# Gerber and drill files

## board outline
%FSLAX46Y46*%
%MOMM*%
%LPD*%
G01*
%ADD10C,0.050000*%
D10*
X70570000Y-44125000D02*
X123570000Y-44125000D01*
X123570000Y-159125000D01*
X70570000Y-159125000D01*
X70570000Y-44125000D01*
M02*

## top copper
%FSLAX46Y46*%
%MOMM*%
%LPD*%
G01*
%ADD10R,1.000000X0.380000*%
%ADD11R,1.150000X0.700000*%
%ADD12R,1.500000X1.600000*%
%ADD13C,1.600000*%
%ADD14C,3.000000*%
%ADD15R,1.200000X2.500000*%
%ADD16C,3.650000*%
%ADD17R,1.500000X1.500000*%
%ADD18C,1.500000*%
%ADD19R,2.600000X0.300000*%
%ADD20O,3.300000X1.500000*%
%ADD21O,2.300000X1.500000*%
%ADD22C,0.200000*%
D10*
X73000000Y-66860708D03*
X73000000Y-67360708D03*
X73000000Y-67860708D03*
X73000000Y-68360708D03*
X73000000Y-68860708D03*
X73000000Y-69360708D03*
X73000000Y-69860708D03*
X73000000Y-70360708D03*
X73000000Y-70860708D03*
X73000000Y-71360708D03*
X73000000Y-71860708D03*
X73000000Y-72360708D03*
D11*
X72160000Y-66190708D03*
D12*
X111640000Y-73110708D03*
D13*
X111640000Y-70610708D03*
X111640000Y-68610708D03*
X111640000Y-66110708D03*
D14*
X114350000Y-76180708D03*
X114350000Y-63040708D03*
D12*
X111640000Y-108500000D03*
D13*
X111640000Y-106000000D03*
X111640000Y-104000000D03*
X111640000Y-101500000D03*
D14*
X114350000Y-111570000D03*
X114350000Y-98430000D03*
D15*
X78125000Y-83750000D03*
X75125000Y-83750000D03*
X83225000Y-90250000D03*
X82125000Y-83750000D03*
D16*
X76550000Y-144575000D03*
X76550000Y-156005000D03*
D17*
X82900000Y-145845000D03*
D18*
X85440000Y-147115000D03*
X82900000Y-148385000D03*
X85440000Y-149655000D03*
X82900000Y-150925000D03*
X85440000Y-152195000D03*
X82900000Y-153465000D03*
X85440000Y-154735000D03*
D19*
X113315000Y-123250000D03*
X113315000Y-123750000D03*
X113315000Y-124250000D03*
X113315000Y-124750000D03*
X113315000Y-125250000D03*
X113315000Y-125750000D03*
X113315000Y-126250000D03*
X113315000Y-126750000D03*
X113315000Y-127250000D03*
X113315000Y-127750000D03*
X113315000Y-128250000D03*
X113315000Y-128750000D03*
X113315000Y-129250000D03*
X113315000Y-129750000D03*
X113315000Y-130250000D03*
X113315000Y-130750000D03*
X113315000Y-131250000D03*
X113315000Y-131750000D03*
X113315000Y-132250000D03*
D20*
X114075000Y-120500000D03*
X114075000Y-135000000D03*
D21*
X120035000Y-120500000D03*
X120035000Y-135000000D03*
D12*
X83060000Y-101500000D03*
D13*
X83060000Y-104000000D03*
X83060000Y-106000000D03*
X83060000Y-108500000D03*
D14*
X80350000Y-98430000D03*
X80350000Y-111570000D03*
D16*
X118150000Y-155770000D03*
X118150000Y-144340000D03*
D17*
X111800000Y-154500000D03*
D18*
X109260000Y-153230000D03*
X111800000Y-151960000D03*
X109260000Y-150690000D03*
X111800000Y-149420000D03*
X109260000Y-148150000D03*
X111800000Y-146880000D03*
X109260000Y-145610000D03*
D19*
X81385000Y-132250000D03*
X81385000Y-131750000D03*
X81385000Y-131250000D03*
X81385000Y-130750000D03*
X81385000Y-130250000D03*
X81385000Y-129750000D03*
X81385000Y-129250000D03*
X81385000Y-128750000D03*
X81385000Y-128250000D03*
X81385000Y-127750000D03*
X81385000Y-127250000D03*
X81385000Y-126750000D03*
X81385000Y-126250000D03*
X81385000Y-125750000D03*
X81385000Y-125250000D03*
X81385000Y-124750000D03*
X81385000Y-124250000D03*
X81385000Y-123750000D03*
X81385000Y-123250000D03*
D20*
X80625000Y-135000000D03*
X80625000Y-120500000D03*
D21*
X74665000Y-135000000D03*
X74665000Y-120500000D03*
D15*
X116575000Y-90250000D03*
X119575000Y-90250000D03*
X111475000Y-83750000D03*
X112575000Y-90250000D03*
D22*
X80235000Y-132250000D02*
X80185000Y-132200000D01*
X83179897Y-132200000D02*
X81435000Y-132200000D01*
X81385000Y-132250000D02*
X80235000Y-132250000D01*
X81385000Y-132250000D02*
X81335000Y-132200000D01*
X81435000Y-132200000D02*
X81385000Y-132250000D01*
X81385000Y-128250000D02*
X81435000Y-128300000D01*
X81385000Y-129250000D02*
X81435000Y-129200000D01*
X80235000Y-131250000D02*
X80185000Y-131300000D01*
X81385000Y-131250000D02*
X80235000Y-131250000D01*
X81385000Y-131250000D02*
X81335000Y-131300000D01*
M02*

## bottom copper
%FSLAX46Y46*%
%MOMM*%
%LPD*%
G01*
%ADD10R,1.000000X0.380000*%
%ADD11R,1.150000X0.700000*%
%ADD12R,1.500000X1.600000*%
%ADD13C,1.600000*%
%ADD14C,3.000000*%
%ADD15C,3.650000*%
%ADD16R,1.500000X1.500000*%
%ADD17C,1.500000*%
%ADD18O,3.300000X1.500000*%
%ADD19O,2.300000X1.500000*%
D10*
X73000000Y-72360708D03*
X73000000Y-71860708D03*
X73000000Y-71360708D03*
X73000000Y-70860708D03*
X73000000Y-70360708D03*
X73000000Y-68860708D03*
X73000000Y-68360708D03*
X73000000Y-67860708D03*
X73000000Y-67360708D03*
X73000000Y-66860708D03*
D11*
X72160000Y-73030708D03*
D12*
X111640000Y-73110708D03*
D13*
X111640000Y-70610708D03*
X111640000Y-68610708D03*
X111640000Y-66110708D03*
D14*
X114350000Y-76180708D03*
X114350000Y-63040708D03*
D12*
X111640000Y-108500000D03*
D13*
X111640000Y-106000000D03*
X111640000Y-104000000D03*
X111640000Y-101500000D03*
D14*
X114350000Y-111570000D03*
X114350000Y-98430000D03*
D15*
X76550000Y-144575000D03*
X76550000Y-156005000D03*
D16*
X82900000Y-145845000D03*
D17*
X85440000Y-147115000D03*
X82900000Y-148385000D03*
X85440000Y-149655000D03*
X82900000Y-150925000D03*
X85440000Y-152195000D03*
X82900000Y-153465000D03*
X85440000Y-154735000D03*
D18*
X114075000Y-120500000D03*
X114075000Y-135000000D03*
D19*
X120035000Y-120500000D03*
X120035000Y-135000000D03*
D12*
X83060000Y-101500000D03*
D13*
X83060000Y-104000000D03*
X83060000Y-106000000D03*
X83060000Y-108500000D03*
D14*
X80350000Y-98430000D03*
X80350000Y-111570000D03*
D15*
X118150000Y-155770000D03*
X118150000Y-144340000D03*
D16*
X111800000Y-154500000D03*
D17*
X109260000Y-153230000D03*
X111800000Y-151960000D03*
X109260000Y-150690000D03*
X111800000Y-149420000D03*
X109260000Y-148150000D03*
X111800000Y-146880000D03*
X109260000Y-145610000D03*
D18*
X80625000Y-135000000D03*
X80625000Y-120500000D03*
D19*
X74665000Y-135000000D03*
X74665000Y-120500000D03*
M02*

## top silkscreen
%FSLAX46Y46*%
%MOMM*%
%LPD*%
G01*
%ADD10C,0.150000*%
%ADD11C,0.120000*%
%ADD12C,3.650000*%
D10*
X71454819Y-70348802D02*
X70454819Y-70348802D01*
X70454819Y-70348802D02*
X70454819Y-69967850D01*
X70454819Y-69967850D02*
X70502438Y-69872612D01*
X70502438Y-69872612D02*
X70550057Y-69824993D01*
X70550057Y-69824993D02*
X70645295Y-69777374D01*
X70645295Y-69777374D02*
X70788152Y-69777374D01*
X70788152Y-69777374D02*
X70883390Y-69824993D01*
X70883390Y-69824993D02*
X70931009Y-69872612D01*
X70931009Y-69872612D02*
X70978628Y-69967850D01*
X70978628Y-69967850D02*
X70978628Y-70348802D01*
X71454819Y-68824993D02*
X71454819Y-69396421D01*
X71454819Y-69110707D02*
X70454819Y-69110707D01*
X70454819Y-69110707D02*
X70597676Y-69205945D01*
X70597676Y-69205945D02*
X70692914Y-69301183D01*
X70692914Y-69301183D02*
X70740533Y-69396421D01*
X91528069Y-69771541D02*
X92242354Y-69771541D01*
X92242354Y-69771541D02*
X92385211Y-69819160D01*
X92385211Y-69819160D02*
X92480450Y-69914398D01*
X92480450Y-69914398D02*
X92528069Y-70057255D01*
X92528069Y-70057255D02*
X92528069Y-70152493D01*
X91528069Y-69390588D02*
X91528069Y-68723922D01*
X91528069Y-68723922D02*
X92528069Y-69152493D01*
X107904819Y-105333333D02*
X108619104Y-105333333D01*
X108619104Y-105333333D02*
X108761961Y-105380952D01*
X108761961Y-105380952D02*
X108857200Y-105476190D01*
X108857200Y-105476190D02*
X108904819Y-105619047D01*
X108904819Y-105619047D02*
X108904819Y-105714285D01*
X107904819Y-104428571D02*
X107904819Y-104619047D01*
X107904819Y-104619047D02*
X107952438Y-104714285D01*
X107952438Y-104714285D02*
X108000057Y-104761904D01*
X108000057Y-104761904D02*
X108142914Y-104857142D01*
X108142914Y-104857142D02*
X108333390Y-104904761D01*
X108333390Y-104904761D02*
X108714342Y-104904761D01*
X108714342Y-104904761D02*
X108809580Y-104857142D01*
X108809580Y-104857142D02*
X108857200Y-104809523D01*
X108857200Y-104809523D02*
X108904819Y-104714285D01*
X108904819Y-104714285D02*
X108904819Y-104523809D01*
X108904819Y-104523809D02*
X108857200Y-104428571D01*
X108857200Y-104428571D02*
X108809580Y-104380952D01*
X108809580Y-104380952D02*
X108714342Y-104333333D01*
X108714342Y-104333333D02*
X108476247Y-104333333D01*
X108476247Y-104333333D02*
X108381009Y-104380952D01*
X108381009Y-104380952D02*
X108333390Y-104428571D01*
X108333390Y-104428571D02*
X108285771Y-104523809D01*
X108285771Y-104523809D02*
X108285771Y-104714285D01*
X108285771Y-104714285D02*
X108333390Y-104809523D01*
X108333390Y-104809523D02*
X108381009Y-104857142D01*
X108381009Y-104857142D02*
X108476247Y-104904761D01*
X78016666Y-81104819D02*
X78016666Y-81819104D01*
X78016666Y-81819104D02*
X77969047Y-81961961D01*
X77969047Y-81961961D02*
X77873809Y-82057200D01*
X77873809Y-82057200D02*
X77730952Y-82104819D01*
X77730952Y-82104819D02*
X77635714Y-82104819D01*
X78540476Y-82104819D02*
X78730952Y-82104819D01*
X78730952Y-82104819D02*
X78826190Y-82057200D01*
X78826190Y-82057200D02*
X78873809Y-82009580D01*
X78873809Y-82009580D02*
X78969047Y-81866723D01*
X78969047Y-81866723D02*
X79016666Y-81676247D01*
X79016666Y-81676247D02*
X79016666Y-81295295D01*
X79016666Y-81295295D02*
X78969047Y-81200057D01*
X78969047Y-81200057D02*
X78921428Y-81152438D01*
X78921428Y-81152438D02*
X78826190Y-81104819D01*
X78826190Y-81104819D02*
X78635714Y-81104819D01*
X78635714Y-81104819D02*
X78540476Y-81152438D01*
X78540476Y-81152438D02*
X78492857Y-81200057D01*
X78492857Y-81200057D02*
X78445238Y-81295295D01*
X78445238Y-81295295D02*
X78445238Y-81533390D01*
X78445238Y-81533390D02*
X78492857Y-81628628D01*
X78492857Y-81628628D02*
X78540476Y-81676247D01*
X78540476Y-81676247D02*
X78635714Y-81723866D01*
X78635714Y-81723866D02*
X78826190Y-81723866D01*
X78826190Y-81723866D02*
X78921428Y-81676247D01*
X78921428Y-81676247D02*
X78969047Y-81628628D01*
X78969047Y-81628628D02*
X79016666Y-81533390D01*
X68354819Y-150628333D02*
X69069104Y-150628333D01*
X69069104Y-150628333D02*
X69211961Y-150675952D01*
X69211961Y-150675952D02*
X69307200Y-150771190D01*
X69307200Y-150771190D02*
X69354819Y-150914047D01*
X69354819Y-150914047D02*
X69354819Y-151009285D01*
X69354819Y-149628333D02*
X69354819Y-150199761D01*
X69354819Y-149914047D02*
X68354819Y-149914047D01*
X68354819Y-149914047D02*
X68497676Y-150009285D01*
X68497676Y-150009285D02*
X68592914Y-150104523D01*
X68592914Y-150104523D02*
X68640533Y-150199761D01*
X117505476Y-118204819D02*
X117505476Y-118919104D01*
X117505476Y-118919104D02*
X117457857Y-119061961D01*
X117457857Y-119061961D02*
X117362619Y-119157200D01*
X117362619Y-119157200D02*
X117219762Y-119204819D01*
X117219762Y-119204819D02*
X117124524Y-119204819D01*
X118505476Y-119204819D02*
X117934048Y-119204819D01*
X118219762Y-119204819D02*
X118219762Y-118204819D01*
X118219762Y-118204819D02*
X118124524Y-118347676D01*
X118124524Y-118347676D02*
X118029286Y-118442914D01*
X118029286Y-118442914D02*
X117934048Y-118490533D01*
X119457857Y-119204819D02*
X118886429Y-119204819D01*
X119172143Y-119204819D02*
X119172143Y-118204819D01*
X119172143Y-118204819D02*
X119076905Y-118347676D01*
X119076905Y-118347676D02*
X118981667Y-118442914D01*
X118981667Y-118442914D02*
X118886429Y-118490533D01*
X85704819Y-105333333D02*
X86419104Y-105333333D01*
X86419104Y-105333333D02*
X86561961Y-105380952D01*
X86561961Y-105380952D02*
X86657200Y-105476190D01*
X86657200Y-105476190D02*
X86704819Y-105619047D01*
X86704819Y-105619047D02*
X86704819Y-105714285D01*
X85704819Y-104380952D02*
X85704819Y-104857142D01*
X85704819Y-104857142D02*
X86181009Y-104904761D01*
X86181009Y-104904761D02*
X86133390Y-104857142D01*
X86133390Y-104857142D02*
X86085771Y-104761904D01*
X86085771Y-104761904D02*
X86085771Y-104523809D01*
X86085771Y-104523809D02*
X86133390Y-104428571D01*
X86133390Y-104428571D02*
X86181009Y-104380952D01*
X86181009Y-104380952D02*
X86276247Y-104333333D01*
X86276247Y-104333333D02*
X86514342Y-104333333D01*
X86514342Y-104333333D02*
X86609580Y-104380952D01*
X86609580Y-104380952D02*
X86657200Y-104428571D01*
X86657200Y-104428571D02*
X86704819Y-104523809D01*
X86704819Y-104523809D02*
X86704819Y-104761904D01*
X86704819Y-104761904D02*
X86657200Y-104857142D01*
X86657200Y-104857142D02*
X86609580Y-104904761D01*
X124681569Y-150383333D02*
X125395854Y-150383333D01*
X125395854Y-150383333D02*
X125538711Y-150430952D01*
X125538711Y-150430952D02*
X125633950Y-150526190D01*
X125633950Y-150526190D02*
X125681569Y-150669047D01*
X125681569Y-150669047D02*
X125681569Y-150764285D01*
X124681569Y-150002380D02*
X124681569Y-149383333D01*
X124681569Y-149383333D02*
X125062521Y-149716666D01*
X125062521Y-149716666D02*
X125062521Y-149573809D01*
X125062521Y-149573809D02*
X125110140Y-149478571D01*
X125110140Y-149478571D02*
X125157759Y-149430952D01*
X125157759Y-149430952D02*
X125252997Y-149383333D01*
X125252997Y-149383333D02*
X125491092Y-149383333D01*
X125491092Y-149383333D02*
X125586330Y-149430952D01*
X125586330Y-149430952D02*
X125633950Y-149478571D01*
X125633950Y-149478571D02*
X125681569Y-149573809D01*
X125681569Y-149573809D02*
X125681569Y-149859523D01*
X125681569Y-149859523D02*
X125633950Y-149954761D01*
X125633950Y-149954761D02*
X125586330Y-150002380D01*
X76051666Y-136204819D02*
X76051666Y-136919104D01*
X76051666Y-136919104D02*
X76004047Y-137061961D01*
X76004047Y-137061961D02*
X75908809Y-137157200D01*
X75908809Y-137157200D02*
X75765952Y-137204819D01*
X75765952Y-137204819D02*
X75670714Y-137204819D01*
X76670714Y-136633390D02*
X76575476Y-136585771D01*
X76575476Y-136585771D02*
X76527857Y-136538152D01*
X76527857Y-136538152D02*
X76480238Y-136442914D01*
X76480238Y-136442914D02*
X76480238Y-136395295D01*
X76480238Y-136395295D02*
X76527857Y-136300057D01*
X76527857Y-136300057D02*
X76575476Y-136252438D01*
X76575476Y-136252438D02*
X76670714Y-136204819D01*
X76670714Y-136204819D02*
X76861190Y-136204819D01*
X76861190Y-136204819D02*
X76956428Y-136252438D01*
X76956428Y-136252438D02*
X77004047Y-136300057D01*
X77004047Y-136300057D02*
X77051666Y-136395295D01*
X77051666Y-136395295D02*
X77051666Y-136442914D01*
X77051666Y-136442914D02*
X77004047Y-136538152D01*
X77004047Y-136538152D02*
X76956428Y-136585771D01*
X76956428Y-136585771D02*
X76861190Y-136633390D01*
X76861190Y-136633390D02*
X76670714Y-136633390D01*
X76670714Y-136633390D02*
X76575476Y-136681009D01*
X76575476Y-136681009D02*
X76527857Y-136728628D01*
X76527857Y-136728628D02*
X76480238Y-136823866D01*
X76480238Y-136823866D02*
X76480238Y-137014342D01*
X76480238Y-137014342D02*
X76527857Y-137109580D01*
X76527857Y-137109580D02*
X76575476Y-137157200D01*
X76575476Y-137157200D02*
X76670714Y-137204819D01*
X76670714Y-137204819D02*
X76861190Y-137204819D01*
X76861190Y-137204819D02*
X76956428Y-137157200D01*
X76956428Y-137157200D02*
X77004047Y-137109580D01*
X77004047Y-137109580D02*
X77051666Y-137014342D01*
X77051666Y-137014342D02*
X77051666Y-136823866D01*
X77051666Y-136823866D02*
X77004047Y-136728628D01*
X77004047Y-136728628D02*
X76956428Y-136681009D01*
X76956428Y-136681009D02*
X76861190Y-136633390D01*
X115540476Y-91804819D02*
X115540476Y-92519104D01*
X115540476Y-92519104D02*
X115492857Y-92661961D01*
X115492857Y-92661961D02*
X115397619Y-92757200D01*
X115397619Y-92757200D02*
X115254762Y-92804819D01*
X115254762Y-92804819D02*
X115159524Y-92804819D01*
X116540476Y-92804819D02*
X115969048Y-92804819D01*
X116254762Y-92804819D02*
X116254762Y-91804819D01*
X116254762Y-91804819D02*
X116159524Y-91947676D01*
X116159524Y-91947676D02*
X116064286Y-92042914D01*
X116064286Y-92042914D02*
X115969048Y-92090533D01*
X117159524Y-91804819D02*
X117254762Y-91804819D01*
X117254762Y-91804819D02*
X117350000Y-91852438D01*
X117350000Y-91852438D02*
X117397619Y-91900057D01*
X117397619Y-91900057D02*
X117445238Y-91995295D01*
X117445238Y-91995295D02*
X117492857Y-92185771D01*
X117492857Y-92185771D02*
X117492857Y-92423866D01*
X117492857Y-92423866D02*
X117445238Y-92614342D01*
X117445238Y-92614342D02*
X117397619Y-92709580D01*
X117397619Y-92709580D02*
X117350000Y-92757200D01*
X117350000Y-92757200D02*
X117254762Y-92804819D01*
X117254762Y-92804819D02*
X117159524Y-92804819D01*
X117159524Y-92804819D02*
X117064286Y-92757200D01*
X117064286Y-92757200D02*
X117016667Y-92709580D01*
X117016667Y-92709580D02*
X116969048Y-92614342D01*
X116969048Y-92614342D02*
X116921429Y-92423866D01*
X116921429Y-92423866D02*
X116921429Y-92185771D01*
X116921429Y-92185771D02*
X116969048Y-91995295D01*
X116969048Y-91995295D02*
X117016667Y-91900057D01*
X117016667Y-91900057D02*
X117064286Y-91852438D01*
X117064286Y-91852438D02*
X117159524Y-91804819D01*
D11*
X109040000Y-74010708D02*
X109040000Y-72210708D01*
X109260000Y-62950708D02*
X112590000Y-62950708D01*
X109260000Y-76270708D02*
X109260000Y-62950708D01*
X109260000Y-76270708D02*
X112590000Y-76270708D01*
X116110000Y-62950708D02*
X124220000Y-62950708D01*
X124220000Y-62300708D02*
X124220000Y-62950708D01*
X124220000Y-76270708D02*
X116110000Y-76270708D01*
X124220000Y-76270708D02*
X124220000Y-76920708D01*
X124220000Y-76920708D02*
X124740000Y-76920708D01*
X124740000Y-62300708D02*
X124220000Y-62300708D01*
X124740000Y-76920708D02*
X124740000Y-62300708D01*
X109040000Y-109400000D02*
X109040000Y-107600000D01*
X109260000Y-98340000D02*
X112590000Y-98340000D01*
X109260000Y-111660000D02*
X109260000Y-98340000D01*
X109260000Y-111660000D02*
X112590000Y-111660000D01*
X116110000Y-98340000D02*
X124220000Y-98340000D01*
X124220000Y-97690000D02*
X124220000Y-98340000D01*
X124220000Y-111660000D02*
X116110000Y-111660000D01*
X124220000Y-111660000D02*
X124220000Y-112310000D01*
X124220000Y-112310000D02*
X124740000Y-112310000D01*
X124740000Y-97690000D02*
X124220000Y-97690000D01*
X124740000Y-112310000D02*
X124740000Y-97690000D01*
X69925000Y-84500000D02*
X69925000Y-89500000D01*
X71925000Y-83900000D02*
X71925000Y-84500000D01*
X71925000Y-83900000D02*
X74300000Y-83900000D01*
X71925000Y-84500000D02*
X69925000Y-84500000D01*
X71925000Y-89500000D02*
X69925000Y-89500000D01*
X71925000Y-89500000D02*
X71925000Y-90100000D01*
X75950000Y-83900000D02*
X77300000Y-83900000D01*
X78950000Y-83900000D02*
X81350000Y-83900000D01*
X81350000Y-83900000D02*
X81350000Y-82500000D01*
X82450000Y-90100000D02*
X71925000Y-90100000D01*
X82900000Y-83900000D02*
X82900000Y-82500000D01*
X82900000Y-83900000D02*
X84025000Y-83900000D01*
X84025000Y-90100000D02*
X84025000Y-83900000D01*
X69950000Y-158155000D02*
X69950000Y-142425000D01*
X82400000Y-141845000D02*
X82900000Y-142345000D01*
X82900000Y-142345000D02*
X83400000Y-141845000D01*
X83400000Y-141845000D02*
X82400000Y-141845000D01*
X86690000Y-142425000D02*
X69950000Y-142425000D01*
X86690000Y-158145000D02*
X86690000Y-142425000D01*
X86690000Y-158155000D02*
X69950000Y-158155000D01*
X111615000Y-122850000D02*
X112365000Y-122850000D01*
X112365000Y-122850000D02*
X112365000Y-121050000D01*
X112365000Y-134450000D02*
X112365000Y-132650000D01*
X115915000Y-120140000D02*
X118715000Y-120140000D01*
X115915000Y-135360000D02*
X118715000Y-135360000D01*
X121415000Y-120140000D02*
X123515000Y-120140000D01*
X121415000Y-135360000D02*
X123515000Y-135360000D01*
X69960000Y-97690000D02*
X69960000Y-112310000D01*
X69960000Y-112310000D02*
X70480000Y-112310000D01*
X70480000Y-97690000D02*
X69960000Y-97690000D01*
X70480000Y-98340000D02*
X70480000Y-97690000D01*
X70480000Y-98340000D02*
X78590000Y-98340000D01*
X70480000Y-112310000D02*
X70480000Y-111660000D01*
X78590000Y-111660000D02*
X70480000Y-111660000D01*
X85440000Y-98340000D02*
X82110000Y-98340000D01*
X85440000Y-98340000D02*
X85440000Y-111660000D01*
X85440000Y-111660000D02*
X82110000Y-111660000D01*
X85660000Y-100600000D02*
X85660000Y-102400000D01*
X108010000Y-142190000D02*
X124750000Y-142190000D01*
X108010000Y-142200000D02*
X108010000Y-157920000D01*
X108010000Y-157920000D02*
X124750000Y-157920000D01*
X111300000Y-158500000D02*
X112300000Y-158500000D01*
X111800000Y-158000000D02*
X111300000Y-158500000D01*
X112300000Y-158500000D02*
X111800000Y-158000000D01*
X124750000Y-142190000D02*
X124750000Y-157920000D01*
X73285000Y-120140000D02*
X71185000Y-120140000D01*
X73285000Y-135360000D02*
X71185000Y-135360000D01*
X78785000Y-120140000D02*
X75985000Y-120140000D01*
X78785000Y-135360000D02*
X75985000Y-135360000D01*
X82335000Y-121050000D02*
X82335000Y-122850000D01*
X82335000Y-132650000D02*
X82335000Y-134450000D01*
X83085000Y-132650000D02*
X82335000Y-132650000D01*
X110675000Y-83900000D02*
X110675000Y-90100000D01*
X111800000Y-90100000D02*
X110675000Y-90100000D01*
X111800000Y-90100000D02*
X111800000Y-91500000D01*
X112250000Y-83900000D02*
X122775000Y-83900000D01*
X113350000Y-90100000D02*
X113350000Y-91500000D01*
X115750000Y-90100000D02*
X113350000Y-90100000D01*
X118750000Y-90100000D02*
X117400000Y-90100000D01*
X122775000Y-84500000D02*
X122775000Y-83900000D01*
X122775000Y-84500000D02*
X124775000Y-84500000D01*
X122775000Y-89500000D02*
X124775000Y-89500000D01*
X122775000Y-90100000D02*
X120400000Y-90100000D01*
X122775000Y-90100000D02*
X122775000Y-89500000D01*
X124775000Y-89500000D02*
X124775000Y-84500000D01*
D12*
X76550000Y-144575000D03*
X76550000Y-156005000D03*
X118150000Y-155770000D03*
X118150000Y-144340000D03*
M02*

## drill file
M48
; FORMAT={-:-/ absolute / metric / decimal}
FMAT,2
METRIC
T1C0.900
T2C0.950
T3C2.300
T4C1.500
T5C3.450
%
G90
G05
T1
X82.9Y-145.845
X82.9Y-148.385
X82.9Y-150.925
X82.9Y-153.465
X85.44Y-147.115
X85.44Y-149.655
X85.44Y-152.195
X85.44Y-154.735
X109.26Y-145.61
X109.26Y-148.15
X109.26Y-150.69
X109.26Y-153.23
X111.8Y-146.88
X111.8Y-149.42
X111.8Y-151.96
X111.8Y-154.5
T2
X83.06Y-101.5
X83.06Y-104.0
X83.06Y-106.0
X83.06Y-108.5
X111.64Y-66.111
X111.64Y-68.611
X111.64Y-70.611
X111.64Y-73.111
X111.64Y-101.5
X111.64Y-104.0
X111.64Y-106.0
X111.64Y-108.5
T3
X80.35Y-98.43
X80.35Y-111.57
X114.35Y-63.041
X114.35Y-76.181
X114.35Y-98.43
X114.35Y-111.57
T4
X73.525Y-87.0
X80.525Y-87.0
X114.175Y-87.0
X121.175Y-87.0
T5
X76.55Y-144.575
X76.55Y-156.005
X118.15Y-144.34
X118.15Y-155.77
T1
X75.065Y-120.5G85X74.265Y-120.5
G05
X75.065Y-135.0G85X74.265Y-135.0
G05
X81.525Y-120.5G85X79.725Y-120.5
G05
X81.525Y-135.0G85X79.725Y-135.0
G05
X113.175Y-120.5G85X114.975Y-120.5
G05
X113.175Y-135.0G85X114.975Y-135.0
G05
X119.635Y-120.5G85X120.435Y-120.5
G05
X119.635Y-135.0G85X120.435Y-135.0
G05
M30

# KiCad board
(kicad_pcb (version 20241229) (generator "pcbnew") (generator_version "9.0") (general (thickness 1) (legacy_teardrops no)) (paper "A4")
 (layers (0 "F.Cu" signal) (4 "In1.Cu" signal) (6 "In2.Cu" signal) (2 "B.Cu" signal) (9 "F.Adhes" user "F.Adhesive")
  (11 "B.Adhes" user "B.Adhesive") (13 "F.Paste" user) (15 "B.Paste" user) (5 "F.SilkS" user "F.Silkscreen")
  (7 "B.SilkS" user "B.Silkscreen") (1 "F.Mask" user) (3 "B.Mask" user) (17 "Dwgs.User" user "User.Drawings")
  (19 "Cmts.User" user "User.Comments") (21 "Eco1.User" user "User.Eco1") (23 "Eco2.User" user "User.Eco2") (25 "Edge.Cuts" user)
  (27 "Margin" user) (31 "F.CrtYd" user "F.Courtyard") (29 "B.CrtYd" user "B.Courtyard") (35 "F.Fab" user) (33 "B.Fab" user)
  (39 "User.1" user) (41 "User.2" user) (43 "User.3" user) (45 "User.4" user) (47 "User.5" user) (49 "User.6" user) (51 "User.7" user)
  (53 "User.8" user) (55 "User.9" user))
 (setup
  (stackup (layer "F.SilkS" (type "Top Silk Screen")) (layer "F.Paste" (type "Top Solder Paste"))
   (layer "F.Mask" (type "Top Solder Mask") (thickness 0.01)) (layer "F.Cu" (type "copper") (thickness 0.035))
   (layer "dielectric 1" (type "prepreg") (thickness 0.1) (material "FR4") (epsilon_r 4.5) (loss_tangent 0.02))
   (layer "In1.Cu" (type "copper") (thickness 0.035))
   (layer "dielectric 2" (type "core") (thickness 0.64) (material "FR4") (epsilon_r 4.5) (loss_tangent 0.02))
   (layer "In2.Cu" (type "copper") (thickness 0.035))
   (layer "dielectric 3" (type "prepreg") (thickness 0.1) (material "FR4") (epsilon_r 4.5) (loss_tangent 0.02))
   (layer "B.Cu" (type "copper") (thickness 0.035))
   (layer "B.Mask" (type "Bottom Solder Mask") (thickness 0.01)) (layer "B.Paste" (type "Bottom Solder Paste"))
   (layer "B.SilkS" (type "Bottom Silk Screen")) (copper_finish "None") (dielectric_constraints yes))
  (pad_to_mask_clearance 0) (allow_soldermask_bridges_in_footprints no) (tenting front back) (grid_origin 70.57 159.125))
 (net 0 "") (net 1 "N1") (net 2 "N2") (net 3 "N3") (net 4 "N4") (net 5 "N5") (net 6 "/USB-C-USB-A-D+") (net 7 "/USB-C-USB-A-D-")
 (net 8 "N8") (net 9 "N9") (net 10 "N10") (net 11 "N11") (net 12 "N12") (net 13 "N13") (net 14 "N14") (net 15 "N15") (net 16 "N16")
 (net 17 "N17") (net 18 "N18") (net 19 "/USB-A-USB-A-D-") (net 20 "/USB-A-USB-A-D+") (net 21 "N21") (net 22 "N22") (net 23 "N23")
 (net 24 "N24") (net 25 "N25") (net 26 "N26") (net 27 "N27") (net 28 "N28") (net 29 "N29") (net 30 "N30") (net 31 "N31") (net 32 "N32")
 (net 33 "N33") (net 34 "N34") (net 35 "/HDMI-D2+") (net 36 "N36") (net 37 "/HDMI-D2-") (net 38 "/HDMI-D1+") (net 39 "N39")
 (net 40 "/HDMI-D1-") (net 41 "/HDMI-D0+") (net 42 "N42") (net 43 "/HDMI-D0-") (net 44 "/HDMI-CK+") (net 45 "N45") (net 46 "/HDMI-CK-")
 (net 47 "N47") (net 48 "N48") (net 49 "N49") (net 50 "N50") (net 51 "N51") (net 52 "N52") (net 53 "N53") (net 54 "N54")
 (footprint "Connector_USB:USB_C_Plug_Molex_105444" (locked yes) (layer "F.Cu") (at 73.04 69.610708 -90)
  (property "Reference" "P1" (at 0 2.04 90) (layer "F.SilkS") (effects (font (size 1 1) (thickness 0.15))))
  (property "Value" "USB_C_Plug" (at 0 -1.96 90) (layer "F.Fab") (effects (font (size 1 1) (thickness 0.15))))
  (pad "A1" smd rect (at -2.75 0.04 270) (size 0.38 1) (layers "F.Cu" "F.Mask" "F.Paste") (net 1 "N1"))
  (pad "A2" smd rect (at -2.25 0.04 270) (size 0.38 1) (layers "F.Cu" "F.Mask" "F.Paste") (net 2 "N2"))
  (pad "A3" smd rect (at -1.75 0.04 270) (size 0.38 1) (layers "F.Cu" "F.Mask" "F.Paste") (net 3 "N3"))
  (pad "A4" smd rect (at -1.25 0.04 270) (size 0.38 1) (layers "F.Cu" "F.Mask" "F.Paste") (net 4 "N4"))
  (pad "A5" smd rect (at -0.75 0.04 270) (size 0.38 1) (layers "F.Cu" "F.Mask" "F.Paste") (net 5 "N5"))
  (pad "A6" smd rect (at -0.25 0.04 270) (size 0.38 1) (layers "F.Cu" "F.Mask" "F.Paste") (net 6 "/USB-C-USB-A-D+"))
  (pad "A7" smd rect (at 0.25 0.04 270) (size 0.38 1) (layers "F.Cu" "F.Mask" "F.Paste") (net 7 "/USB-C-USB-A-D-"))
  (pad "A8" smd rect (at 0.75 0.04 270) (size 0.38 1) (layers "F.Cu" "F.Mask" "F.Paste") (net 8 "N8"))
  (pad "A9" smd rect (at 1.25 0.04 270) (size 0.38 1) (layers "F.Cu" "F.Mask" "F.Paste") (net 4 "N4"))
  (pad "A10" smd rect (at 1.75 0.04 270) (size 0.38 1) (layers "F.Cu" "F.Mask" "F.Paste") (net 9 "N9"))
  (pad "A11" smd rect (at 2.25 0.04 270) (size 0.38 1) (layers "F.Cu" "F.Mask" "F.Paste") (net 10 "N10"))
  (pad "A12" smd rect (at 2.75 0.04 270) (size 0.38 1) (layers "F.Cu" "F.Mask" "F.Paste") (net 1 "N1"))
  (pad "B1" smd rect (at 2.75 0.04 270) (size 0.38 1) (layers "B.Cu" "B.Mask" "B.Paste") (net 1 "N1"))
  (pad "B2" smd rect (at 2.25 0.04 270) (size 0.38 1) (layers "B.Cu" "B.Mask" "B.Paste") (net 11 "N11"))
  (pad "B3" smd rect (at 1.75 0.04 270) (size 0.38 1) (layers "B.Cu" "B.Mask" "B.Paste") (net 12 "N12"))
  (pad "B4" smd rect (at 1.25 0.04 270) (size 0.38 1) (layers "B.Cu" "B.Mask" "B.Paste") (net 4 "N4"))
  (pad "B5" smd rect (at 0.75 0.04 270) (size 0.38 1) (layers "B.Cu" "B.Mask" "B.Paste") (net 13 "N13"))
  (pad "B8" smd rect (at -0.75 0.04 270) (size 0.38 1) (layers "B.Cu" "B.Mask" "B.Paste") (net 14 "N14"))
  (pad "B9" smd rect (at -1.25 0.04 270) (size 0.38 1) (layers "B.Cu" "B.Mask" "B.Paste") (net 4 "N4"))
  (pad "B10" smd rect (at -1.75 0.04 270) (size 0.38 1) (layers "B.Cu" "B.Mask" "B.Paste") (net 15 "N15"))
  (pad "B11" smd rect (at -2.25 0.04 270) (size 0.38 1) (layers "B.Cu" "B.Mask" "B.Paste") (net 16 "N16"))
  (pad "B12" smd rect (at -2.75 0.04 270) (size 0.38 1) (layers "B.Cu" "B.Mask" "B.Paste") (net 1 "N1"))
  (pad "S1" smd rect (at -3.42 0.88 270) (size 0.7 1.15) (layers "F.Cu" "F.Mask" "F.Paste") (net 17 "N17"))
  (pad "S1" smd rect (at 3.42 0.88 270) (size 0.7 1.15) (layers "B.Cu" "B.Mask" "B.Paste") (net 17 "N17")))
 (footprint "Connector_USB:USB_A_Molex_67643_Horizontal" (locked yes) (layer "F.Cu") (at 111.64 73.110708 90)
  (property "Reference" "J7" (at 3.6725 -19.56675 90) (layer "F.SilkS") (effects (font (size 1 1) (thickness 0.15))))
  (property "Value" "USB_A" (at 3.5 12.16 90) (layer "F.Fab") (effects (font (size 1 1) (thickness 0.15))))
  (fp_line (start -0.9 -2.6) (end 0.9 -2.6) (stroke (width 0.12) (type solid)) (layer "F.SilkS"))
  (fp_line (start 10.16 -2.38) (end 10.16 0.95) (stroke (width 0.12) (type solid)) (layer "F.SilkS"))
  (fp_line (start -3.16 -2.38) (end 10.16 -2.38) (stroke (width 0.12) (type solid)) (layer "F.SilkS"))
  (fp_line (start -3.16 -2.38) (end -3.16 0.95) (stroke (width 0.12) (type solid)) (layer "F.SilkS"))
  (fp_line (start 10.16 4.47) (end 10.16 12.58) (stroke (width 0.12) (type solid)) (layer "F.SilkS"))
  (fp_line (start 10.81 12.58) (end 10.16 12.58) (stroke (width 0.12) (type solid)) (layer "F.SilkS"))
  (fp_line (start -3.16 12.58) (end -3.16 4.47) (stroke (width 0.12) (type solid)) (layer "F.SilkS"))
  (fp_line (start -3.16 12.58) (end -3.81 12.58) (stroke (width 0.12) (type solid)) (layer "F.SilkS"))
  (fp_line (start -3.81 12.58) (end -3.81 13.1) (stroke (width 0.12) (type solid)) (layer "F.SilkS"))
  (fp_line (start 10.81 13.1) (end 10.81 12.58) (stroke (width 0.12) (type solid)) (layer "F.SilkS"))
  (fp_line (start -3.81 13.1) (end 10.81 13.1) (stroke (width 0.12) (type solid)) (layer "F.SilkS"))
  (pad "1" thru_hole rect (at 0 0 90) (size 1.6 1.5) (drill 0.95) (layers "*.Cu" "*.Mask") (remove_unused_layers no) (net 4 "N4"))
  (pad "2" thru_hole circle (at 2.5 0 90) (size 1.6 1.6) (drill 0.95) (layers "*.Cu" "*.Mask") (remove_unused_layers no)
   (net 7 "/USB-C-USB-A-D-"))
  (pad "3" thru_hole circle (at 4.5 0 90) (size 1.6 1.6) (drill 0.95) (layers "*.Cu" "*.Mask") (remove_unused_layers no)
   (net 6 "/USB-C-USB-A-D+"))
  (pad "4" thru_hole circle (at 7 0 90) (size 1.6 1.6) (drill 0.95) (layers "*.Cu" "*.Mask") (remove_unused_layers no) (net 1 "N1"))
  (pad "5" thru_hole circle (at -3.07 2.71 90) (size 3 3) (drill 2.3) (layers "*.Cu" "*.Mask") (remove_unused_layers no) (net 17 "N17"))
  (pad "5" thru_hole circle (at 10.07 2.71 90) (size 3 3) (drill 2.3) (layers "*.Cu" "*.Mask") (remove_unused_layers no) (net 17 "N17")))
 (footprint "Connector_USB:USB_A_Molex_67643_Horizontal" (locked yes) (layer "F.Cu") (at 111.64 108.5 90)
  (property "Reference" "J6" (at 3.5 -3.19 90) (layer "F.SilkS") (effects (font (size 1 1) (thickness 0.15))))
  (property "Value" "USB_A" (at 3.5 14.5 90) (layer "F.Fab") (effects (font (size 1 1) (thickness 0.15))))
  (fp_line (start -0.9 -2.6) (end 0.9 -2.6) (stroke (width 0.12) (type solid)) (layer "F.SilkS"))
  (fp_line (start 10.16 -2.38) (end 10.16 0.95) (stroke (width 0.12) (type solid)) (layer "F.SilkS"))
  (fp_line (start -3.16 -2.38) (end 10.16 -2.38) (stroke (width 0.12) (type solid)) (layer "F.SilkS"))
  (fp_line (start -3.16 -2.38) (end -3.16 0.95) (stroke (width 0.12) (type solid)) (layer "F.SilkS"))
  (fp_line (start 10.16 4.47) (end 10.16 12.58) (stroke (width 0.12) (type solid)) (layer "F.SilkS"))
  (fp_line (start 10.81 12.58) (end 10.16 12.58) (stroke (width 0.12) (type solid)) (layer "F.SilkS"))
  (fp_line (start -3.16 12.58) (end -3.16 4.47) (stroke (width 0.12) (type solid)) (layer "F.SilkS"))
  (fp_line (start -3.16 12.58) (end -3.81 12.58) (stroke (width 0.12) (type solid)) (layer "F.SilkS"))
  (fp_line (start -3.81 12.58) (end -3.81 13.1) (stroke (width 0.12) (type solid)) (layer "F.SilkS"))
  (fp_line (start 10.81 13.1) (end 10.81 12.58) (stroke (width 0.12) (type solid)) (layer "F.SilkS"))
  (fp_line (start -3.81 13.1) (end 10.81 13.1) (stroke (width 0.12) (type solid)) (layer "F.SilkS"))
  (pad "1" thru_hole rect (at 0 0 90) (size 1.6 1.5) (drill 0.95) (layers "*.Cu" "*.Mask") (remove_unused_layers no) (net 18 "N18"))
  (pad "2" thru_hole circle (at 2.5 0 90) (size 1.6 1.6) (drill 0.95) (layers "*.Cu" "*.Mask") (remove_unused_layers no)
   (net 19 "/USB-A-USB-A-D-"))
  (pad "3" thru_hole circle (at 4.5 0 90) (size 1.6 1.6) (drill 0.95) (layers "*.Cu" "*.Mask") (remove_unused_layers no)
   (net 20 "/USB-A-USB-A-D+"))
  (pad "4" thru_hole circle (at 7 0 90) (size 1.6 1.6) (drill 0.95) (layers "*.Cu" "*.Mask") (remove_unused_layers no) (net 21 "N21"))
  (pad "5" thru_hole circle (at -3.07 2.71 90) (size 3 3) (drill 2.3) (layers "*.Cu" "*.Mask") (remove_unused_layers no) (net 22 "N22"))
  (pad "5" thru_hole circle (at 10.07 2.71 90) (size 3 3) (drill 2.3) (layers "*.Cu" "*.Mask") (remove_unused_layers no) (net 22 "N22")))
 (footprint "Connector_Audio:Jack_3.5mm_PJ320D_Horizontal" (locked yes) (layer "F.Cu") (at 78.3 87)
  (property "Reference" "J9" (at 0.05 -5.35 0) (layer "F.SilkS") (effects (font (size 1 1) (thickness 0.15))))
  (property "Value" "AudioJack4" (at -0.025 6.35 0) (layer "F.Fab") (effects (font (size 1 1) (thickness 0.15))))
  (fp_line (start -8.375 -2.5) (end -8.375 2.5) (stroke (width 0.12) (type solid)) (layer "F.SilkS"))
  (fp_line (start -6.375 -3.1) (end -6.375 -2.5) (stroke (width 0.12) (type solid)) (layer "F.SilkS"))
  (fp_line (start -6.375 -3.1) (end -4 -3.1) (stroke (width 0.12) (type solid)) (layer "F.SilkS"))
  (fp_line (start -6.375 -2.5) (end -8.375 -2.5) (stroke (width 0.12) (type solid)) (layer "F.SilkS"))
  (fp_line (start -6.375 2.5) (end -8.375 2.5) (stroke (width 0.12) (type solid)) (layer "F.SilkS"))
  (fp_line (start -6.375 2.5) (end -6.375 3.1) (stroke (width 0.12) (type solid)) (layer "F.SilkS"))
  (fp_line (start -2.35 -3.1) (end -1 -3.1) (stroke (width 0.12) (type solid)) (layer "F.SilkS"))
  (fp_line (start 0.65 -3.1) (end 3.05 -3.1) (stroke (width 0.12) (type solid)) (layer "F.SilkS"))
  (fp_line (start 3.05 -3.1) (end 3.05 -4.5) (stroke (width 0.12) (type solid)) (layer "F.SilkS"))
  (fp_line (start 4.15 3.1) (end -6.375 3.1) (stroke (width 0.12) (type solid)) (layer "F.SilkS"))
  (fp_line (start 4.6 -3.1) (end 4.6 -4.5) (stroke (width 0.12) (type solid)) (layer "F.SilkS"))
  (fp_line (start 4.6 -3.1) (end 5.725 -3.1) (stroke (width 0.12) (type solid)) (layer "F.SilkS"))
  (fp_line (start 5.725 3.1) (end 5.725 -3.1) (stroke (width 0.12) (type solid)) (layer "F.SilkS"))
  (pad "" np_thru_hole circle (at -4.775 0) (size 1.5 1.5) (drill 1.5) (layers "*.Cu" "*.Mask"))
  (pad "" np_thru_hole circle (at 2.225 0) (size 1.5 1.5) (drill 1.5) (layers "*.Cu" "*.Mask"))
  (pad "R1" smd rect (at -0.175 -3.25) (size 1.2 2.5) (layers "F.Cu" "F.Mask" "F.Paste") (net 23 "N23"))
  (pad "R2" smd rect (at -3.175 -3.25) (size 1.2 2.5) (layers "F.Cu" "F.Mask" "F.Paste") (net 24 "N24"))
  (pad "S" smd rect (at 4.925 3.25) (size 1.2 2.5) (layers "F.Cu" "F.Mask" "F.Paste") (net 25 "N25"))
  (pad "T" smd rect (at 3.825 -3.25) (size 1.2 2.5) (layers "F.Cu" "F.Mask" "F.Paste") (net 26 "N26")))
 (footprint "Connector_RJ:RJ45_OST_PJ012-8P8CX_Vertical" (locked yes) (layer "F.Cu") (at 82.9 145.845 -90)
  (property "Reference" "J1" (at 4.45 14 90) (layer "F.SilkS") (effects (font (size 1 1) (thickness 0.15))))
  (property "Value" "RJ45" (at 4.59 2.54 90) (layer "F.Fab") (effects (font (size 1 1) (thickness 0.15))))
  (fp_line (start 12.31 12.95) (end -3.42 12.95) (stroke (width 0.12) (type solid)) (layer "F.SilkS"))
  (fp_line (start -4 0.5) (end -3.5 0) (stroke (width 0.12) (type solid)) (layer "F.SilkS"))
  (fp_line (start -3.5 0) (end -4 -0.5) (stroke (width 0.12) (type solid)) (layer "F.SilkS"))
  (fp_line (start -4 -0.5) (end -4 0.5) (stroke (width 0.12) (type solid)) (layer "F.SilkS"))
  (fp_line (start -3.42 -3.79) (end -3.42 12.95) (stroke (width 0.12) (type solid)) (layer "F.SilkS"))
  (fp_line (start 12.3 -3.79) (end -3.42 -3.79) (stroke (width 0.12) (type solid)) (layer "F.SilkS"))
  (fp_line (start 12.31 -3.79) (end 12.31 12.95) (stroke (width 0.12) (type solid)) (layer "F.SilkS"))
  (pad "" np_thru_hole circle (at -1.27 6.35 270) (size 3.65 3.65) (drill 3.45) (layers "*.Cu" "*.SilkS" "*.Mask"))
  (pad "" np_thru_hole circle (at 10.16 6.35 270) (size 3.65 3.65) (drill 3.45) (layers "*.Cu" "*.SilkS" "*.Mask"))
  (pad "1" thru_hole rect (at 0 0 270) (size 1.5 1.5) (drill 0.9) (layers "*.Cu" "*.Mask") (remove_unused_layers no) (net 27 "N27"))
  (pad "2" thru_hole circle (at 1.27 -2.54 270) (size 1.5 1.5) (drill 0.9) (layers "*.Cu" "*.Mask") (remove_unused_layers no) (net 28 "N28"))
  (pad "3" thru_hole circle (at 2.54 0 270) (size 1.5 1.5) (drill 0.9) (layers "*.Cu" "*.Mask") (remove_unused_layers no) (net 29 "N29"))
  (pad "4" thru_hole circle (at 3.81 -2.54 270) (size 1.5 1.5) (drill 0.9) (layers "*.Cu" "*.Mask") (remove_unused_layers no) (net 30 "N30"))
  (pad "5" thru_hole circle (at 5.08 0 270) (size 1.5 1.5) (drill 0.9) (layers "*.Cu" "*.Mask") (remove_unused_layers no) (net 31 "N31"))
  (pad "6" thru_hole circle (at 6.35 -2.54 270) (size 1.5 1.5) (drill 0.9) (layers "*.Cu" "*.Mask") (remove_unused_layers no) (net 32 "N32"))
  (pad "7" thru_hole circle (at 7.62 0 270) (size 1.5 1.5) (drill 0.9) (layers "*.Cu" "*.Mask") (remove_unused_layers no) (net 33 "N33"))
  (pad "8" thru_hole circle (at 8.89 -2.54 270) (size 1.5 1.5) (drill 0.9) (layers "*.Cu" "*.Mask") (remove_unused_layers no) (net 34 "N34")))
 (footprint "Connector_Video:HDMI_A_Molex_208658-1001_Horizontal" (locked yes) (layer "F.Cu") (at 116.6 127.75)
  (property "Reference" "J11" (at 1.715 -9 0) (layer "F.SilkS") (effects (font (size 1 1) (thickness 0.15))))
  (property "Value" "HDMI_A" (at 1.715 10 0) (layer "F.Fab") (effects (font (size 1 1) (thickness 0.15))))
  (fp_line (start -4.985 -4.9) (end -4.235 -4.9) (stroke (width 0.12) (type solid)) (layer "F.SilkS"))
  (fp_line (start -4.235 -4.9) (end -4.235 -6.7) (stroke (width 0.12) (type solid)) (layer "F.SilkS"))
  (fp_line (start -4.235 6.7) (end -4.235 4.9) (stroke (width 0.12) (type solid)) (layer "F.SilkS"))
  (fp_line (start -0.685 -7.61) (end 2.115 -7.61) (stroke (width 0.12) (type solid)) (layer "F.SilkS"))
  (fp_line (start -0.685 7.61) (end 2.115 7.61) (stroke (width 0.12) (type solid)) (layer "F.SilkS"))
  (fp_line (start 4.815 -7.61) (end 6.915 -7.61) (stroke (width 0.12) (type solid)) (layer "F.SilkS"))
  (fp_line (start 4.815 7.61) (end 6.915 7.61) (stroke (width 0.12) (type solid)) (layer "F.SilkS"))
  (pad "1" smd rect (at -3.285 -4.5) (size 2.6 0.3) (layers "F.Cu" "F.Mask" "F.Paste") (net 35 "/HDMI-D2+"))
  (pad "2" smd rect (at -3.285 -4) (size 2.6 0.3) (layers "F.Cu" "F.Mask" "F.Paste") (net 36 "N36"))
  (pad "3" smd rect (at -3.285 -3.5) (size 2.6 0.3) (layers "F.Cu" "F.Mask" "F.Paste") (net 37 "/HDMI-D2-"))
  (pad "4" smd rect (at -3.285 -3) (size 2.6 0.3) (layers "F.Cu" "F.Mask" "F.Paste") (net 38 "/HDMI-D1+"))
  (pad "5" smd rect (at -3.285 -2.5) (size 2.6 0.3) (layers "F.Cu" "F.Mask" "F.Paste") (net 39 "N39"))
  (pad "6" smd rect (at -3.285 -2) (size 2.6 0.3) (layers "F.Cu" "F.Mask" "F.Paste") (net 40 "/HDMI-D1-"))
  (pad "7" smd rect (at -3.285 -1.5) (size 2.6 0.3) (layers "F.Cu" "F.Mask" "F.Paste") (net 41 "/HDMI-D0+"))
  (pad "8" smd rect (at -3.285 -1) (size 2.6 0.3) (layers "F.Cu" "F.Mask" "F.Paste") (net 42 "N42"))
  (pad "9" smd rect (at -3.285 -0.5) (size 2.6 0.3) (layers "F.Cu" "F.Mask" "F.Paste") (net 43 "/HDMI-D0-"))
  (pad "10" smd rect (at -3.285 0) (size 2.6 0.3) (layers "F.Cu" "F.Mask" "F.Paste") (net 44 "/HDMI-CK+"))
  (pad "11" smd rect (at -3.285 0.5) (size 2.6 0.3) (layers "F.Cu" "F.Mask" "F.Paste") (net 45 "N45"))
  (pad "12" smd rect (at -3.285 1) (size 2.6 0.3) (layers "F.Cu" "F.Mask" "F.Paste") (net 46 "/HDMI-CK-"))
  (pad "13" smd rect (at -3.285 1.5) (size 2.6 0.3) (layers "F.Cu" "F.Mask" "F.Paste") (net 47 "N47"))
  (pad "14" smd rect (at -3.285 2) (size 2.6 0.3) (layers "F.Cu" "F.Mask" "F.Paste") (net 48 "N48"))
  (pad "15" smd rect (at -3.285 2.5) (size 2.6 0.3) (layers "F.Cu" "F.Mask" "F.Paste") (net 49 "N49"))
  (pad "16" smd rect (at -3.285 3) (size 2.6 0.3) (layers "F.Cu" "F.Mask" "F.Paste") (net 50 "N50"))
  (pad "17" smd rect (at -3.285 3.5) (size 2.6 0.3) (layers "F.Cu" "F.Mask" "F.Paste") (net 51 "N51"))
  (pad "18" smd rect (at -3.285 4) (size 2.6 0.3) (layers "F.Cu" "F.Mask" "F.Paste") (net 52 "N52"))
  (pad "19" smd rect (at -3.285 4.5) (size 2.6 0.3) (layers "F.Cu" "F.Mask" "F.Paste") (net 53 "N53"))
  (pad "SH" thru_hole oval (at -2.525 -7.25) (size 3.3 1.5) (drill oval 2.7 0.9) (layers "*.Cu" "*.Mask") (remove_unused_layers no)
   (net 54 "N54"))
  (pad "SH" thru_hole oval (at -2.525 7.25) (size 3.3 1.5) (drill oval 2.7 0.9) (layers "*.Cu" "*.Mask") (remove_unused_layers no)
   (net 54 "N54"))
  (pad "SH" thru_hole oval (at 3.435 -7.25) (size 2.3 1.5) (drill oval 1.7 0.9) (layers "*.Cu" "*.Mask") (remove_unused_layers no)
   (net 54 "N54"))
  (pad "SH" thru_hole oval (at 3.435 7.25) (size 2.3 1.5) (drill oval 1.7 0.9) (layers "*.Cu" "*.Mask") (remove_unused_layers no)
   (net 54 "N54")))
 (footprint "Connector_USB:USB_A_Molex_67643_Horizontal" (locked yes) (layer "F.Cu") (at 83.06 101.5 -90)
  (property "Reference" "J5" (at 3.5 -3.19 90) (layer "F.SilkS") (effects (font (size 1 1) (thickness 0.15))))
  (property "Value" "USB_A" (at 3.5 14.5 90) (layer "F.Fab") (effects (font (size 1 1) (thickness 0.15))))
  (fp_line (start -3.81 13.1) (end 10.81 13.1) (stroke (width 0.12) (type solid)) (layer "F.SilkS"))
  (fp_line (start 10.81 13.1) (end 10.81 12.58) (stroke (width 0.12) (type solid)) (layer "F.SilkS"))
  (fp_line (start -3.81 12.58) (end -3.81 13.1) (stroke (width 0.12) (type solid)) (layer "F.SilkS"))
  (fp_line (start -3.16 12.58) (end -3.81 12.58) (stroke (width 0.12) (type solid)) (layer "F.SilkS"))
  (fp_line (start -3.16 12.58) (end -3.16 4.47) (stroke (width 0.12) (type solid)) (layer "F.SilkS"))
  (fp_line (start 10.81 12.58) (end 10.16 12.58) (stroke (width 0.12) (type solid)) (layer "F.SilkS"))
  (fp_line (start 10.16 4.47) (end 10.16 12.58) (stroke (width 0.12) (type solid)) (layer "F.SilkS"))
  (fp_line (start -3.16 -2.38) (end -3.16 0.95) (stroke (width 0.12) (type solid)) (layer "F.SilkS"))
  (fp_line (start -3.16 -2.38) (end 10.16 -2.38) (stroke (width 0.12) (type solid)) (layer "F.SilkS"))
  (fp_line (start 10.16 -2.38) (end 10.16 0.95) (stroke (width 0.12) (type solid)) (layer "F.SilkS"))
  (fp_line (start -0.9 -2.6) (end 0.9 -2.6) (stroke (width 0.12) (type solid)) (layer "F.SilkS"))
  (pad "1" thru_hole rect (at 0 0 270) (size 1.6 1.5) (drill 0.95) (layers "*.Cu" "*.Mask") (remove_unused_layers no) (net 18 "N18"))
  (pad "2" thru_hole circle (at 2.5 0 270) (size 1.6 1.6) (drill 0.95) (layers "*.Cu" "*.Mask") (remove_unused_layers no)
   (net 19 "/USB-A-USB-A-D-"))
  (pad "3" thru_hole circle (at 4.5 0 270) (size 1.6 1.6) (drill 0.95) (layers "*.Cu" "*.Mask") (remove_unused_layers no)
   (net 20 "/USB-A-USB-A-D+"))
  (pad "4" thru_hole circle (at 7 0 270) (size 1.6 1.6) (drill 0.95) (layers "*.Cu" "*.Mask") (remove_unused_layers no) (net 21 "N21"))
  (pad "5" thru_hole circle (at -3.07 2.71 270) (size 3 3) (drill 2.3) (layers "*.Cu" "*.Mask") (remove_unused_layers no) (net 22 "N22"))
  (pad "5" thru_hole circle (at 10.07 2.71 270) (size 3 3) (drill 2.3) (layers "*.Cu" "*.Mask") (remove_unused_layers no) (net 22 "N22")))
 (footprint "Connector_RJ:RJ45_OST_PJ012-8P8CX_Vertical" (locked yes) (layer "F.Cu") (at 111.8 154.5 90)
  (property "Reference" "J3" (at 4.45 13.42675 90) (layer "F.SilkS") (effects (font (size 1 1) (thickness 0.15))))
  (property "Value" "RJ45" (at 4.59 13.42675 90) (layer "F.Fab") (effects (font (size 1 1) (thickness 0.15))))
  (fp_line (start 12.31 -3.79) (end 12.31 12.95) (stroke (width 0.12) (type solid)) (layer "F.SilkS"))
  (fp_line (start 12.3 -3.79) (end -3.42 -3.79) (stroke (width 0.12) (type solid)) (layer "F.SilkS"))
  (fp_line (start -3.42 -3.79) (end -3.42 12.95) (stroke (width 0.12) (type solid)) (layer "F.SilkS"))
  (fp_line (start -4 -0.5) (end -4 0.5) (stroke (width 0.12) (type solid)) (layer "F.SilkS"))
  (fp_line (start -3.5 0) (end -4 -0.5) (stroke (width 0.12) (type solid)) (layer "F.SilkS"))
  (fp_line (start -4 0.5) (end -3.5 0) (stroke (width 0.12) (type solid)) (layer "F.SilkS"))
  (fp_line (start 12.31 12.95) (end -3.42 12.95) (stroke (width 0.12) (type solid)) (layer "F.SilkS"))
  (pad "" np_thru_hole circle (at -1.27 6.35 90) (size 3.65 3.65) (drill 3.45) (layers "*.Cu" "*.SilkS" "*.Mask"))
  (pad "" np_thru_hole circle (at 10.16 6.35 90) (size 3.65 3.65) (drill 3.45) (layers "*.Cu" "*.SilkS" "*.Mask"))
  (pad "1" thru_hole rect (at 0 0 90) (size 1.5 1.5) (drill 0.9) (layers "*.Cu" "*.Mask") (remove_unused_layers no) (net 27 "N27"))
  (pad "2" thru_hole circle (at 1.27 -2.54 90) (size 1.5 1.5) (drill 0.9) (layers "*.Cu" "*.Mask") (remove_unused_layers no) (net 28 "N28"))
  (pad "3" thru_hole circle (at 2.54 0 90) (size 1.5 1.5) (drill 0.9) (layers "*.Cu" "*.Mask") (remove_unused_layers no) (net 29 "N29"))
  (pad "4" thru_hole circle (at 3.81 -2.54 90) (size 1.5 1.5) (drill 0.9) (layers "*.Cu" "*.Mask") (remove_unused_layers no) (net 30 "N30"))
  (pad "5" thru_hole circle (at 5.08 0 90) (size 1.5 1.5) (drill 0.9) (layers "*.Cu" "*.Mask") (remove_unused_layers no) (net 31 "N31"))
  (pad "6" thru_hole circle (at 6.35 -2.54 90) (size 1.5 1.5) (drill 0.9) (layers "*.Cu" "*.Mask") (remove_unused_layers no) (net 32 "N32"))
  (pad "7" thru_hole circle (at 7.62 0 90) (size 1.5 1.5) (drill 0.9) (layers "*.Cu" "*.Mask") (remove_unused_layers no) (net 33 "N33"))
  (pad "8" thru_hole circle (at 8.89 -2.54 90) (size 1.5 1.5) (drill 0.9) (layers "*.Cu" "*.Mask") (remove_unused_layers no) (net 34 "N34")))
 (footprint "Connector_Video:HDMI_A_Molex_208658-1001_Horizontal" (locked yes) (layer "F.Cu") (at 78.1 127.75 180)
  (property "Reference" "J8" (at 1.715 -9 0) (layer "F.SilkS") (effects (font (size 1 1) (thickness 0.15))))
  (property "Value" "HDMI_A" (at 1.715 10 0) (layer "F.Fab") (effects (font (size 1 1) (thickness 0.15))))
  (fp_line (start 4.815 7.61) (end 6.915 7.61) (stroke (width 0.12) (type solid)) (layer "F.SilkS"))
  (fp_line (start 4.815 -7.61) (end 6.915 -7.61) (stroke (width 0.12) (type solid)) (layer "F.SilkS"))
  (fp_line (start -0.685 7.61) (end 2.115 7.61) (stroke (width 0.12) (type solid)) (layer "F.SilkS"))
  (fp_line (start -0.685 -7.61) (end 2.115 -7.61) (stroke (width 0.12) (type solid)) (layer "F.SilkS"))
  (fp_line (start -4.235 6.7) (end -4.235 4.9) (stroke (width 0.12) (type solid)) (layer "F.SilkS"))
  (fp_line (start -4.235 -4.9) (end -4.235 -6.7) (stroke (width 0.12) (type solid)) (layer "F.SilkS"))
  (fp_line (start -4.985 -4.9) (end -4.235 -4.9) (stroke (width 0.12) (type solid)) (layer "F.SilkS"))
  (pad "1" smd rect (at -3.285 -4.5 180) (size 2.6 0.3) (layers "F.Cu" "F.Mask" "F.Paste") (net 35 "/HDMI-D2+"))
  (pad "2" smd rect (at -3.285 -4 180) (size 2.6 0.3) (layers "F.Cu" "F.Mask" "F.Paste") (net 36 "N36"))
  (pad "3" smd rect (at -3.285 -3.5 180) (size 2.6 0.3) (layers "F.Cu" "F.Mask" "F.Paste") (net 37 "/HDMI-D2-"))
  (pad "4" smd rect (at -3.285 -3 180) (size 2.6 0.3) (layers "F.Cu" "F.Mask" "F.Paste") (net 38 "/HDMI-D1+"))
  (pad "5" smd rect (at -3.285 -2.5 180) (size 2.6 0.3) (layers "F.Cu" "F.Mask" "F.Paste") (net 39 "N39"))
  (pad "6" smd rect (at -3.285 -2 180) (size 2.6 0.3) (layers "F.Cu" "F.Mask" "F.Paste") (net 40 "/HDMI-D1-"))
  (pad "7" smd rect (at -3.285 -1.5 180) (size 2.6 0.3) (layers "F.Cu" "F.Mask" "F.Paste") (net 41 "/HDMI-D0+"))
  (pad "8" smd rect (at -3.285 -1 180) (size 2.6 0.3) (layers "F.Cu" "F.Mask" "F.Paste") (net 42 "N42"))
  (pad "9" smd rect (at -3.285 -0.5 180) (size 2.6 0.3) (layers "F.Cu" "F.Mask" "F.Paste") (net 43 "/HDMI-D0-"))
  (pad "10" smd rect (at -3.285 0 180) (size 2.6 0.3) (layers "F.Cu" "F.Mask" "F.Paste") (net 44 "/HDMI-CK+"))
  (pad "11" smd rect (at -3.285 0.5 180) (size 2.6 0.3) (layers "F.Cu" "F.Mask" "F.Paste") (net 45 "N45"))
  (pad "12" smd rect (at -3.285 1 180) (size 2.6 0.3) (layers "F.Cu" "F.Mask" "F.Paste") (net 46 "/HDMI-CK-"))
  (pad "13" smd rect (at -3.285 1.5 180) (size 2.6 0.3) (layers "F.Cu" "F.Mask" "F.Paste") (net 47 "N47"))
  (pad "14" smd rect (at -3.285 2 180) (size 2.6 0.3) (layers "F.Cu" "F.Mask" "F.Paste") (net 48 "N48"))
  (pad "15" smd rect (at -3.285 2.5 180) (size 2.6 0.3) (layers "F.Cu" "F.Mask" "F.Paste") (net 49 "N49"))
  (pad "16" smd rect (at -3.285 3 180) (size 2.6 0.3) (layers "F.Cu" "F.Mask" "F.Paste") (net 50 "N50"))
  (pad "17" smd rect (at -3.285 3.5 180) (size 2.6 0.3) (layers "F.Cu" "F.Mask" "F.Paste") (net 51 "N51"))
  (pad "18" smd rect (at -3.285 4 180) (size 2.6 0.3) (layers "F.Cu" "F.Mask" "F.Paste") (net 52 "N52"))
  (pad "19" smd rect (at -3.285 4.5 180) (size 2.6 0.3) (layers "F.Cu" "F.Mask" "F.Paste") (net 53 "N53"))
  (pad "SH" thru_hole oval (at -2.525 -7.25 180) (size 3.3 1.5) (drill oval 2.7 0.9) (layers "*.Cu" "*.Mask") (remove_unused_layers no)
   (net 54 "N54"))
  (pad "SH" thru_hole oval (at -2.525 7.25 180) (size 3.3 1.5) (drill oval 2.7 0.9) (layers "*.Cu" "*.Mask") (remove_unused_layers no)
   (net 54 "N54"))
  (pad "SH" thru_hole oval (at 3.435 -7.25 180) (size 2.3 1.5) (drill oval 1.7 0.9) (layers "*.Cu" "*.Mask") (remove_unused_layers no)
   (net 54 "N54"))
  (pad "SH" thru_hole oval (at 3.435 7.25 180) (size 2.3 1.5) (drill oval 1.7 0.9) (layers "*.Cu" "*.Mask") (remove_unused_layers no)
   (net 54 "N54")))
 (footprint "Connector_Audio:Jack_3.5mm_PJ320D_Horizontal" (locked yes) (layer "F.Cu") (at 116.4 87 180)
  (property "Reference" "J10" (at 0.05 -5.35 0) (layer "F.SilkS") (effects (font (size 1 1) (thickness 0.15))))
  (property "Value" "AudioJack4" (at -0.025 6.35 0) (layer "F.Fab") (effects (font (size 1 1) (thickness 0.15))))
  (fp_line (start 5.725 3.1) (end 5.725 -3.1) (stroke (width 0.12) (type solid)) (layer "F.SilkS"))
  (fp_line (start 4.6 -3.1) (end 5.725 -3.1) (stroke (width 0.12) (type solid)) (layer "F.SilkS"))
  (fp_line (start 4.6 -3.1) (end 4.6 -4.5) (stroke (width 0.12) (type solid)) (layer "F.SilkS"))
  (fp_line (start 4.15 3.1) (end -6.375 3.1) (stroke (width 0.12) (type solid)) (layer "F.SilkS"))
  (fp_line (start 3.05 -3.1) (end 3.05 -4.5) (stroke (width 0.12) (type solid)) (layer "F.SilkS"))
  (fp_line (start 0.65 -3.1) (end 3.05 -3.1) (stroke (width 0.12) (type solid)) (layer "F.SilkS"))
  (fp_line (start -2.35 -3.1) (end -1 -3.1) (stroke (width 0.12) (type solid)) (layer "F.SilkS"))
  (fp_line (start -6.375 2.5) (end -6.375 3.1) (stroke (width 0.12) (type solid)) (layer "F.SilkS"))
  (fp_line (start -6.375 2.5) (end -8.375 2.5) (stroke (width 0.12) (type solid)) (layer "F.SilkS"))
  (fp_line (start -6.375 -2.5) (end -8.375 -2.5) (stroke (width 0.12) (type solid)) (layer "F.SilkS"))
  (fp_line (start -6.375 -3.1) (end -4 -3.1) (stroke (width 0.12) (type solid)) (layer "F.SilkS"))
  (fp_line (start -6.375 -3.1) (end -6.375 -2.5) (stroke (width 0.12) (type solid)) (layer "F.SilkS"))
  (fp_line (start -8.375 -2.5) (end -8.375 2.5) (stroke (width 0.12) (type solid)) (layer "F.SilkS"))
  (pad "" np_thru_hole circle (at -4.775 0 180) (size 1.5 1.5) (drill 1.5) (layers "*.Cu" "*.Mask"))
  (pad "" np_thru_hole circle (at 2.225 0 180) (size 1.5 1.5) (drill 1.5) (layers "*.Cu" "*.Mask"))
  (pad "R1" smd rect (at -0.175 -3.25 180) (size 1.2 2.5) (layers "F.Cu" "F.Mask" "F.Paste") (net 23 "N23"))
  (pad "R2" smd rect (at -3.175 -3.25 180) (size 1.2 2.5) (layers "F.Cu" "F.Mask" "F.Paste") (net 24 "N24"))
  (pad "S" smd rect (at 4.925 3.25 180) (size 1.2 2.5) (layers "F.Cu" "F.Mask" "F.Paste") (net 25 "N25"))
  (pad "T" smd rect (at 3.825 -3.25 180) (size 1.2 2.5) (layers "F.Cu" "F.Mask" "F.Paste") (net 26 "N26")))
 (gr_rect (start 70.57 44.125) (end 123.57 159.125) (stroke (width 0.05) (type default)) (fill no) (layer "Edge.Cuts"))
 (segment (start 80.235 132.25) (end 80.185 132.2) (width 0.2) (layer "F.Cu") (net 35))
 (segment (start 83.179897 132.2) (end 81.435 132.2) (width 0.2) (layer "F.Cu") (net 35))
 (segment (start 81.385 132.25) (end 80.235 132.25) (width 0.2) (layer "F.Cu") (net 35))
 (segment (start 81.385 132.25) (end 81.335 132.2) (width 0.2) (layer "F.Cu") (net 35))
 (segment (start 81.435 132.2) (end 81.385 132.25) (width 0.2) (layer "F.Cu") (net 35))
 (segment (start 81.385 128.25) (end 81.435 128.3) (width 0.2) (layer "F.Cu") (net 43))
 (segment (start 81.385 129.25) (end 81.435 129.2) (width 0.2) (layer "F.Cu") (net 41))
 (segment (start 80.235 131.25) (end 80.185 131.3) (width 0.2) (layer "F.Cu") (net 37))
 (segment (start 81.385 131.25) (end 80.235 131.25) (width 0.2) (layer "F.Cu") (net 37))
 (segment (start 81.385 131.25) (end 81.335 131.3) (width 0.2) (layer "F.Cu") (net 37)))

